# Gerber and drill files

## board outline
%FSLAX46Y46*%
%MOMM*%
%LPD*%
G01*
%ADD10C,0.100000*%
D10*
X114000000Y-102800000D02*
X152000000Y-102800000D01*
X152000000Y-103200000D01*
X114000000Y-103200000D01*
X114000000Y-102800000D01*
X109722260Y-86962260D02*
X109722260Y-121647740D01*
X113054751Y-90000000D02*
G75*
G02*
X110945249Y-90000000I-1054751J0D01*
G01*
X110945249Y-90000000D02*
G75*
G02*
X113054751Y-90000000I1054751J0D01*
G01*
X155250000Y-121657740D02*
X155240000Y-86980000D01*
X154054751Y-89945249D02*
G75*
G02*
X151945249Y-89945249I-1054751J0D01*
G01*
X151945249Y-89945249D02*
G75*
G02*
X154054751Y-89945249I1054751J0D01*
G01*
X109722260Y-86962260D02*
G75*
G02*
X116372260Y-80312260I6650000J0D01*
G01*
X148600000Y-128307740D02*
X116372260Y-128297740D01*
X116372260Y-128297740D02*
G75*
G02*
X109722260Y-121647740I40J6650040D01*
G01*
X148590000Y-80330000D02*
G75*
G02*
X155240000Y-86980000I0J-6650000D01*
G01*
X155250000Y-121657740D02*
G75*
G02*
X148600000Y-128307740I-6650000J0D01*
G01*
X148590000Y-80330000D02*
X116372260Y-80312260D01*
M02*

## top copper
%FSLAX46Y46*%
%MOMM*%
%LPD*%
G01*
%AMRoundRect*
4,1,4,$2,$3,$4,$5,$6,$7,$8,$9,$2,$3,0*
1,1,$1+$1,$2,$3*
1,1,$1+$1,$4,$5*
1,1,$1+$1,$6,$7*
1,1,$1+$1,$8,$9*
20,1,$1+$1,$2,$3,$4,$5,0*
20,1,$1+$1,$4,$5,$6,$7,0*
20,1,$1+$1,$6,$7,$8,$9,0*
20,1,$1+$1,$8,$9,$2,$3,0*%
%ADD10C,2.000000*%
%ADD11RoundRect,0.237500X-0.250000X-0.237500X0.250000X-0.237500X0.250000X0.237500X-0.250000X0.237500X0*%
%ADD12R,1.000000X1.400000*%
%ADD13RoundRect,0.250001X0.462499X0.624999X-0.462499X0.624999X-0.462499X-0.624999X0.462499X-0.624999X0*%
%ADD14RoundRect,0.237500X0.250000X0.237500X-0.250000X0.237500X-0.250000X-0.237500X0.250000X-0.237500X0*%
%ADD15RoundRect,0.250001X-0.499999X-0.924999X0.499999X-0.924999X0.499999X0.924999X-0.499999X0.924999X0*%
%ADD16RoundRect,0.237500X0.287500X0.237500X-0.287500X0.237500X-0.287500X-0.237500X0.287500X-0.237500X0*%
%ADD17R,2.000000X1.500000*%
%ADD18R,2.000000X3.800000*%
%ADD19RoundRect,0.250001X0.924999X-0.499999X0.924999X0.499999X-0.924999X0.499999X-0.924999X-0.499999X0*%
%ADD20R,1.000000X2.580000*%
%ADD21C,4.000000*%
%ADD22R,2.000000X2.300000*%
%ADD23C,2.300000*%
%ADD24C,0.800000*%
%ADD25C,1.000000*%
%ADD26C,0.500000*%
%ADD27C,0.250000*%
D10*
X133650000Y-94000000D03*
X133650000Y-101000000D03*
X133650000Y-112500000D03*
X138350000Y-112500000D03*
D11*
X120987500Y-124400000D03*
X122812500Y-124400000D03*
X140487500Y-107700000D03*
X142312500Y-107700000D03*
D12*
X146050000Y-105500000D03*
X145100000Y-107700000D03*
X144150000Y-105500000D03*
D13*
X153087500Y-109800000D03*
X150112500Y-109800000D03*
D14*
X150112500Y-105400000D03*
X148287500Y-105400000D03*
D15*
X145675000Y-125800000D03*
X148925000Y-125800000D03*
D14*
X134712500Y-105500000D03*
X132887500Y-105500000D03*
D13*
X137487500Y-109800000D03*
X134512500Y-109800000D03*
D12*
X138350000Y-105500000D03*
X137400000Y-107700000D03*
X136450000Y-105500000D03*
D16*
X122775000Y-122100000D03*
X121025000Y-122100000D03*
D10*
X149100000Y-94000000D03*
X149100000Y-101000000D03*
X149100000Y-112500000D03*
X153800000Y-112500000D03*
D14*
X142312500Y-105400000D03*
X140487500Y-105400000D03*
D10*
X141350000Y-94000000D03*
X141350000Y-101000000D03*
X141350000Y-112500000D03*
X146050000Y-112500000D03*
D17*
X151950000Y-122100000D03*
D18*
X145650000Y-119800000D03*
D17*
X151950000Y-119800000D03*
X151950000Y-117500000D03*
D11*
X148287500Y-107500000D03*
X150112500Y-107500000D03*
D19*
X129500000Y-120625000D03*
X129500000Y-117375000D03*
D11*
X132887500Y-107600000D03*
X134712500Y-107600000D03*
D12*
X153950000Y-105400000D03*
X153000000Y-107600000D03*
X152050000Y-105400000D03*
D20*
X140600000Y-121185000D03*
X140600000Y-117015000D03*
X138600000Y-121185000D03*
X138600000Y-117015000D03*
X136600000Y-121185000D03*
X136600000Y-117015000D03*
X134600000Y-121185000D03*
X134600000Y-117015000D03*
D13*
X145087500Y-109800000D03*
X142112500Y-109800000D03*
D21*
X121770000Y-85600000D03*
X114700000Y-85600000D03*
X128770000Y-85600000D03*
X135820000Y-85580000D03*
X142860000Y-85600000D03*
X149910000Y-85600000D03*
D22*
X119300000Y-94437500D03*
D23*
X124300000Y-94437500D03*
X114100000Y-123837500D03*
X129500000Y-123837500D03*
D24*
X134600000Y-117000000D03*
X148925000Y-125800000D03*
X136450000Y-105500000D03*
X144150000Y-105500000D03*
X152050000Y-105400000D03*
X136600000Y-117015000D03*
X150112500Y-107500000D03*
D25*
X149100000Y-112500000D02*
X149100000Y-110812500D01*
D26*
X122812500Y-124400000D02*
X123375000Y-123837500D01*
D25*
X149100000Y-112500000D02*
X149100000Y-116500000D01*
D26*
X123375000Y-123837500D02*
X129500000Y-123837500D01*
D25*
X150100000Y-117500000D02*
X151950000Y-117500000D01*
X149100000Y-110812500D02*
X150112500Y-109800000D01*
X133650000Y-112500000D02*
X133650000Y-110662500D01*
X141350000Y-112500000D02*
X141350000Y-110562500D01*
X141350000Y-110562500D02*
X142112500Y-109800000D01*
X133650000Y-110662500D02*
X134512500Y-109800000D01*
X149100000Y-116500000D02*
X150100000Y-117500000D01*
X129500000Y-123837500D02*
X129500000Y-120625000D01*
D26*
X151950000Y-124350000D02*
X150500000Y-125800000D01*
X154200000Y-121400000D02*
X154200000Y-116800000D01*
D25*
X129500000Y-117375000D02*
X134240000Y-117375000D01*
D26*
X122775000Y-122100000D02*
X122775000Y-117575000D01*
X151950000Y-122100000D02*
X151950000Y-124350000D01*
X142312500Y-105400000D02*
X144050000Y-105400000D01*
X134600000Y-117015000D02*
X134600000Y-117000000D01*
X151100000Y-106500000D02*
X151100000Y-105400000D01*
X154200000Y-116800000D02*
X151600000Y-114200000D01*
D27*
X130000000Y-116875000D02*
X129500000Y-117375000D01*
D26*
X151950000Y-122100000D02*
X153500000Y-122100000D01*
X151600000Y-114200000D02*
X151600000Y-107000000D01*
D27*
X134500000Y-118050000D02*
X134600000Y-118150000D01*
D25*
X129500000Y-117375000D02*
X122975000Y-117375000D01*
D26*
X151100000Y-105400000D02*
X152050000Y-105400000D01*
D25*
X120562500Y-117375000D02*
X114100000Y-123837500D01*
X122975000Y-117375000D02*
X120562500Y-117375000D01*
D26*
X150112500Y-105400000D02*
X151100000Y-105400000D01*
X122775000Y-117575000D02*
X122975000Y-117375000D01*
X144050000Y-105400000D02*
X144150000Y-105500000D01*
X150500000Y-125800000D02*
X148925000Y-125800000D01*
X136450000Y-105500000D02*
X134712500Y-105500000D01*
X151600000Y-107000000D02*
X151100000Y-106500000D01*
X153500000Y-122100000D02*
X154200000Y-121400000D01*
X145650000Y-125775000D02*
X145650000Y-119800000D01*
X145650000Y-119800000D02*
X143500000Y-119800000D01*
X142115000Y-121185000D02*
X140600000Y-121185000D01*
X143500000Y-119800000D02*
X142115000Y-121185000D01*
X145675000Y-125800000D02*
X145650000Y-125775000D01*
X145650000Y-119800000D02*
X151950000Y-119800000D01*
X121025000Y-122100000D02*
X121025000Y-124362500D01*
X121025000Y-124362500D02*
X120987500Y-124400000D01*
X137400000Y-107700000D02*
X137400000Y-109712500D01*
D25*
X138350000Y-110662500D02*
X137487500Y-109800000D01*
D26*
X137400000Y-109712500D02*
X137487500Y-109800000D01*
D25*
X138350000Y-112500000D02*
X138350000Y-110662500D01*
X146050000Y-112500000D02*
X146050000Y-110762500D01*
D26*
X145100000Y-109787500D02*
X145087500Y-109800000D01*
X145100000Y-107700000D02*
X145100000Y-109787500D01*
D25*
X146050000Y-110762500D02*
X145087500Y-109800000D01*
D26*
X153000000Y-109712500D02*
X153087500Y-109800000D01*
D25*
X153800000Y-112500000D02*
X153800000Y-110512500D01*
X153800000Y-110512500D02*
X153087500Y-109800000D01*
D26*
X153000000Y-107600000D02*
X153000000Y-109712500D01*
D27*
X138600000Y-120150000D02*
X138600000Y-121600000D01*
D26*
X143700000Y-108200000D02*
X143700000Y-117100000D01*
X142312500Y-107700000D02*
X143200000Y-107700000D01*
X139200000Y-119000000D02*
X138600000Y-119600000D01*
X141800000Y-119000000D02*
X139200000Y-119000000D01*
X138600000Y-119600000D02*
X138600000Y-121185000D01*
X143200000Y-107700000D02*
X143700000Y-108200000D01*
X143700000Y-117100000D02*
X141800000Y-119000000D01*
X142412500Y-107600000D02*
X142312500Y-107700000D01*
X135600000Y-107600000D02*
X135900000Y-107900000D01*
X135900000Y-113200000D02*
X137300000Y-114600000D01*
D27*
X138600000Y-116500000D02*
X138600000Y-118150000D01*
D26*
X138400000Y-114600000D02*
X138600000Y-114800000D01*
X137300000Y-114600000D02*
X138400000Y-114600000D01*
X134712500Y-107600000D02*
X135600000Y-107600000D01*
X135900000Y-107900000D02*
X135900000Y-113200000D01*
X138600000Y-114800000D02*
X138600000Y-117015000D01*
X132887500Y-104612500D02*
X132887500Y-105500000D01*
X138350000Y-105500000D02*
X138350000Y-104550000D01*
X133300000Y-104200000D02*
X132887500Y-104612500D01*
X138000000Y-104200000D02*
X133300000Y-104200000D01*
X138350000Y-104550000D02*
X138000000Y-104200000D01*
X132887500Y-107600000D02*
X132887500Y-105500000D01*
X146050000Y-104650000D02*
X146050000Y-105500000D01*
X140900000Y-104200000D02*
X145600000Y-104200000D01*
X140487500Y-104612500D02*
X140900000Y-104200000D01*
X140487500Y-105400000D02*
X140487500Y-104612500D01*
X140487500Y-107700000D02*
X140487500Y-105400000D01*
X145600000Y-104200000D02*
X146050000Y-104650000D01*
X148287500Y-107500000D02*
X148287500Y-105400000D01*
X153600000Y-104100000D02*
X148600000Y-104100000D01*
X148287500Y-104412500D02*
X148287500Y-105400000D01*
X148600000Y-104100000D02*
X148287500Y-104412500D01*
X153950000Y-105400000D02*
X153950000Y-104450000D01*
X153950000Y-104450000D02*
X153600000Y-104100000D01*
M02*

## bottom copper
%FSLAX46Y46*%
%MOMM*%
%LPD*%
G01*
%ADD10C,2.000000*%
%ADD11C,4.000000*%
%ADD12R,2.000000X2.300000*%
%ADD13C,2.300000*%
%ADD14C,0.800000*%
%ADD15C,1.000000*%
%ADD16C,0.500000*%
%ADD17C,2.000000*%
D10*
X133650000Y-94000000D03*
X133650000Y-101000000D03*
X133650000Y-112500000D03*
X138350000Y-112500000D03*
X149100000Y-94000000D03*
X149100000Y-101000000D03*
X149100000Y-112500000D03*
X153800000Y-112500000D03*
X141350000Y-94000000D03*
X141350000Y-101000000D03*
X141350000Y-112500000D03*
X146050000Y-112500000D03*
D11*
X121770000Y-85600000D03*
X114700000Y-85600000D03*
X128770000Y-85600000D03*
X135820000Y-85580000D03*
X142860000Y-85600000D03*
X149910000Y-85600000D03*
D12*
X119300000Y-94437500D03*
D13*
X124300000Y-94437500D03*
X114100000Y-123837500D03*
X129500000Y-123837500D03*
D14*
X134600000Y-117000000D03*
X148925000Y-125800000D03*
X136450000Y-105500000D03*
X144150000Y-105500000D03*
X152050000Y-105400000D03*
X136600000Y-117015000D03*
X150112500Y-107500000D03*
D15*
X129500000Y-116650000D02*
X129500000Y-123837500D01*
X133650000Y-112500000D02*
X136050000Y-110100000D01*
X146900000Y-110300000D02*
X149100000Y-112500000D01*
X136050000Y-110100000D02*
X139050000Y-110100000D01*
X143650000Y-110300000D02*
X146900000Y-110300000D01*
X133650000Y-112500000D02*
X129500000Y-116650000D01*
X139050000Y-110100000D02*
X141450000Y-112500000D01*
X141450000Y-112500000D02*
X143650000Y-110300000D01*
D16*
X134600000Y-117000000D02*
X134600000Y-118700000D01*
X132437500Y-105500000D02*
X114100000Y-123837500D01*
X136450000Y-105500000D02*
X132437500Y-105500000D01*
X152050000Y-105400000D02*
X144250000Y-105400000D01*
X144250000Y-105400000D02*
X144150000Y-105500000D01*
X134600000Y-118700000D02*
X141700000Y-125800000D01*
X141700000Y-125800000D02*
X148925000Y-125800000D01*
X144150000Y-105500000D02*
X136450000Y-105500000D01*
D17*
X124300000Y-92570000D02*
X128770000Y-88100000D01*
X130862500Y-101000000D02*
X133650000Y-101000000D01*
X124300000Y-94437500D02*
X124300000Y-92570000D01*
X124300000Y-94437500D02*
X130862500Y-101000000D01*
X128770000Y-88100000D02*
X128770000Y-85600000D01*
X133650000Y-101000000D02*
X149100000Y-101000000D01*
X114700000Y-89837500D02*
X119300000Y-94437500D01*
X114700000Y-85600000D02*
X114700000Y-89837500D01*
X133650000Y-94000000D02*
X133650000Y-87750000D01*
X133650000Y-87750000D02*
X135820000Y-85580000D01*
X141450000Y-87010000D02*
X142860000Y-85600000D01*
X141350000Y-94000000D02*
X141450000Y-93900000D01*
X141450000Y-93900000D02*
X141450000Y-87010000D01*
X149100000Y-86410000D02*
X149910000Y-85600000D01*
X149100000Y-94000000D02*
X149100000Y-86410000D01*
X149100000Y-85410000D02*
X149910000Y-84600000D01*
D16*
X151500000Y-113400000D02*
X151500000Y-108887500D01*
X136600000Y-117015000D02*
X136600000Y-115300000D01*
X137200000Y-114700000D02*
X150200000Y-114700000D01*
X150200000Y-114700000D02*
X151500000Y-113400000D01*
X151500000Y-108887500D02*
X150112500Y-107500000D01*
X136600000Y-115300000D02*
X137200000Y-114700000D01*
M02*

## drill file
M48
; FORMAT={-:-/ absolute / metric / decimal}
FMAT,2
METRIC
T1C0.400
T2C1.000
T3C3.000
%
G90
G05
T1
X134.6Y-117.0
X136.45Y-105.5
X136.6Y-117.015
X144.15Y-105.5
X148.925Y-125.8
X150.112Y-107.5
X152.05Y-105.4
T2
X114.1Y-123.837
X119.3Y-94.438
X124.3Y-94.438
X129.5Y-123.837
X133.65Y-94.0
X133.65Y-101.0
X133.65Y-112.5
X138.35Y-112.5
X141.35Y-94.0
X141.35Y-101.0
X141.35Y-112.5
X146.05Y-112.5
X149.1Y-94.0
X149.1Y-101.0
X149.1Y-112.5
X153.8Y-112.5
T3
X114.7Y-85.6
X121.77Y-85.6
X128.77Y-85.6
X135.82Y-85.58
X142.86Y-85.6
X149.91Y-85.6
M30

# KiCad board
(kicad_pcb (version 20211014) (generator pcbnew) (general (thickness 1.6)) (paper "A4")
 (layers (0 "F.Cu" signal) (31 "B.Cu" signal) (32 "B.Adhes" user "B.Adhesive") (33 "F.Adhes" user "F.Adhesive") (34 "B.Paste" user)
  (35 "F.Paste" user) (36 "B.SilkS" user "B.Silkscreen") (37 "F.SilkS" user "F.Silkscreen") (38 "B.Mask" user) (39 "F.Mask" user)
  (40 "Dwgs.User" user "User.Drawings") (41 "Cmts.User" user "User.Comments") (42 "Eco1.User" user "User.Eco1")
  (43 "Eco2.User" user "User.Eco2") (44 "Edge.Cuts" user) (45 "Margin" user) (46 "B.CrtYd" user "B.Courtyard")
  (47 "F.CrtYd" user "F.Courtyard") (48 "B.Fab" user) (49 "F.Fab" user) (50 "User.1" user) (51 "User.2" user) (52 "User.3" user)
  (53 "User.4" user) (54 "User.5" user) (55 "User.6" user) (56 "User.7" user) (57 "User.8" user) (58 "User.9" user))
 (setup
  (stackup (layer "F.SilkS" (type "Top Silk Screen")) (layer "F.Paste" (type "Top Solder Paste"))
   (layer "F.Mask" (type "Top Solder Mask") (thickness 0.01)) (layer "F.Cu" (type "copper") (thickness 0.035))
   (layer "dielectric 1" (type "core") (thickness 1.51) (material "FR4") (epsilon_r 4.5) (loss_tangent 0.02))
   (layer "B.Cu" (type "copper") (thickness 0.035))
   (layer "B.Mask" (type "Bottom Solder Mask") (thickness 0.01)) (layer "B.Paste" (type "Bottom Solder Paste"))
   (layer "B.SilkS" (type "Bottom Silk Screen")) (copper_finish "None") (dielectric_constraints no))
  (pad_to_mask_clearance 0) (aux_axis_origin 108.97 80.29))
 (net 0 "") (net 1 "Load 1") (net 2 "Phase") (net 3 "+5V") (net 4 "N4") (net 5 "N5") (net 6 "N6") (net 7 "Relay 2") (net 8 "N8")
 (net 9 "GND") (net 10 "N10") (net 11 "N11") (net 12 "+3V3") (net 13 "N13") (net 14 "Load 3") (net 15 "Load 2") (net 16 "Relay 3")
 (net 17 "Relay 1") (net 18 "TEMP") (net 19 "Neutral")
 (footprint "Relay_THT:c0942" (layer "F.Cu") (at 133.65 101 90)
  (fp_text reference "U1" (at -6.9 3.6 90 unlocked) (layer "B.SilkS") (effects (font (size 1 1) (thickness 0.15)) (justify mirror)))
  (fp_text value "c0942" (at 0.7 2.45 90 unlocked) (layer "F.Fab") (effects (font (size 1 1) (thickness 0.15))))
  (pad "1" thru_hole circle (at 7 0 90) (size 2 2) (drill 1) (layers *.Cu *.Mask) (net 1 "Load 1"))
  (pad "2" thru_hole circle (at 0 0 90) (size 2 2) (drill 1) (layers *.Cu *.Mask) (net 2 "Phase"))
  (pad "3" thru_hole circle (at -11.5 0 90) (size 2 2) (drill 1) (layers *.Cu *.Mask) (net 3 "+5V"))
  (pad "4" thru_hole circle (at -11.5 4.7 90) (size 2 2) (drill 1) (layers *.Cu *.Mask) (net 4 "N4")))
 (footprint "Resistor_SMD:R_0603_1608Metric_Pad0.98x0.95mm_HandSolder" (layer "F.Cu") (at 121.9 124.4)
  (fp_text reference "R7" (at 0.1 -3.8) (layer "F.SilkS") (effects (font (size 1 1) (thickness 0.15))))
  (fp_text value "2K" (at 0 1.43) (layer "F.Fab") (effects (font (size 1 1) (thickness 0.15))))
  (pad "1" smd roundrect (at -0.9125 0) (size 0.975 0.95) (layers "F.Cu" "F.Paste" "F.Mask") (roundrect_rratio 0.25) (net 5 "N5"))
  (pad "2" smd roundrect (at 0.9125 0) (size 0.975 0.95) (layers "F.Cu" "F.Paste" "F.Mask") (roundrect_rratio 0.25) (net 3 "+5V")))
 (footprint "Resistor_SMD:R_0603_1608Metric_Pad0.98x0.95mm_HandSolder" (layer "F.Cu") (at 141.4 107.7)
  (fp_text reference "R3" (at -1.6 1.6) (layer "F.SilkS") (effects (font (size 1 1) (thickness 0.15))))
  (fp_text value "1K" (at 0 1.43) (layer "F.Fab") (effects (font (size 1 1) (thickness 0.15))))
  (pad "1" smd roundrect (at -0.9125 0) (size 0.975 0.95) (layers "F.Cu" "F.Paste" "F.Mask") (roundrect_rratio 0.25) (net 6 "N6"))
  (pad "2" smd roundrect (at 0.9125 0) (size 0.975 0.95) (layers "F.Cu" "F.Paste" "F.Mask") (roundrect_rratio 0.25) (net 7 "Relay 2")))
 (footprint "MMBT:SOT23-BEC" (layer "F.Cu") (at 145.1 106.6 180)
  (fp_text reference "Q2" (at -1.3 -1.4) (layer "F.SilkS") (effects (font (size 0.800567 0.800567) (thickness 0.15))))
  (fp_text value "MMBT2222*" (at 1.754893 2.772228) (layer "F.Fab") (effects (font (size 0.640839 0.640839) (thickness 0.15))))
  (pad "B" smd rect locked (at -0.95 1.1 180) (size 1 1.4) (layers "F.Cu" "F.Paste" "F.Mask") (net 6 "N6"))
  (pad "C" smd rect locked (at 0 -1.1 180) (size 1 1.4) (layers "F.Cu" "F.Paste" "F.Mask") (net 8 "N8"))
  (pad "E" smd rect locked (at 0.95 1.1 180) (size 1 1.4) (layers "F.Cu" "F.Paste" "F.Mask") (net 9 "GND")))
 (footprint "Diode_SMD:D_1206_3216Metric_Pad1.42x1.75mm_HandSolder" (layer "F.Cu") (at 151.6 109.8 180)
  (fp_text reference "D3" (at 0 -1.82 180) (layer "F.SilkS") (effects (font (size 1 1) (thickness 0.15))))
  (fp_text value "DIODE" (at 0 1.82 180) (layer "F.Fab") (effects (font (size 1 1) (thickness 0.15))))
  (pad "1" smd roundrect (at -1.4875 0 180) (size 1.425 1.75) (layers "F.Cu" "F.Paste" "F.Mask") (roundrect_rratio 0.175439) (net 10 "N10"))
  (pad "2" smd roundrect (at 1.4875 0 180) (size 1.425 1.75) (layers "F.Cu" "F.Paste" "F.Mask") (roundrect_rratio 0.175439) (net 3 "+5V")))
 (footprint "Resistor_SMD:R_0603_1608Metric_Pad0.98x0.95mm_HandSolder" (layer "F.Cu") (at 149.2 105.4 180)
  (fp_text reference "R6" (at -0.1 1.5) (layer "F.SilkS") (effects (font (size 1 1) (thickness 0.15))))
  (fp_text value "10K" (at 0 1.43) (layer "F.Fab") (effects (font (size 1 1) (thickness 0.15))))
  (pad "1" smd roundrect (at -0.9125 0 180) (size 0.975 0.95) (layers "F.Cu" "F.Paste" "F.Mask") (roundrect_rratio 0.25) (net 9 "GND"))
  (pad "2" smd roundrect (at 0.9125 0 180) (size 0.975 0.95) (layers "F.Cu" "F.Paste" "F.Mask") (roundrect_rratio 0.25) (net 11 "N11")))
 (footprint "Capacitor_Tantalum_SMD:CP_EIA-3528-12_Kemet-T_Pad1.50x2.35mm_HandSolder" (layer "F.Cu") (at 147.3 125.8)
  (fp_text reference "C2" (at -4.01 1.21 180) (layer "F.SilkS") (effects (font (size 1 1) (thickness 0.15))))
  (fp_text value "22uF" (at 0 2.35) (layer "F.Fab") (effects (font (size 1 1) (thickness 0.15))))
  (pad "1" smd roundrect (at -1.625 0) (size 1.5 2.35) (layers "F.Cu" "F.Paste" "F.Mask") (roundrect_rratio 0.166667) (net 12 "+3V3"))
  (pad "2" smd roundrect (at 1.625 0) (size 1.5 2.35) (layers "F.Cu" "F.Paste" "F.Mask") (roundrect_rratio 0.166667) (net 9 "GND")))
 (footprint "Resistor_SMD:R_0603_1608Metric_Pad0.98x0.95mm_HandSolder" (layer "F.Cu") (at 133.8 105.5 180)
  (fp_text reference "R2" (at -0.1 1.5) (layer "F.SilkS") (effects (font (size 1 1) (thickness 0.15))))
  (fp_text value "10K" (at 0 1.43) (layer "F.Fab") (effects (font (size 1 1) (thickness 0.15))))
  (pad "1" smd roundrect (at -0.9125 0 180) (size 0.975 0.95) (layers "F.Cu" "F.Paste" "F.Mask") (roundrect_rratio 0.25) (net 9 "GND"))
  (pad "2" smd roundrect (at 0.9125 0 180) (size 0.975 0.95) (layers "F.Cu" "F.Paste" "F.Mask") (roundrect_rratio 0.25) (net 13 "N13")))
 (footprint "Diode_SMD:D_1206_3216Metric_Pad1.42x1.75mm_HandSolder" (layer "F.Cu") (at 136 109.8 180)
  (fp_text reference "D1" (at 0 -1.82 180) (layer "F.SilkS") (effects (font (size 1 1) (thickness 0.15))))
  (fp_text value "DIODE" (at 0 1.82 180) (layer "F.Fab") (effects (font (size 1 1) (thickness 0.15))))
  (pad "1" smd roundrect (at -1.4875 0 180) (size 1.425 1.75) (layers "F.Cu" "F.Paste" "F.Mask") (roundrect_rratio 0.175439) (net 4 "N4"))
  (pad "2" smd roundrect (at 1.4875 0 180) (size 1.425 1.75) (layers "F.Cu" "F.Paste" "F.Mask") (roundrect_rratio 0.175439) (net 3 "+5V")))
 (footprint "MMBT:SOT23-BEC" (layer "F.Cu") (at 137.4 106.6 180)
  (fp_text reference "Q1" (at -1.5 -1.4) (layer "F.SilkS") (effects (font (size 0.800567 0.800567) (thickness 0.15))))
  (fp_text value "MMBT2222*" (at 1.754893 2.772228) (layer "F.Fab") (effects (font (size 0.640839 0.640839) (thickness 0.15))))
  (pad "B" smd rect locked (at -0.95 1.1 180) (size 1 1.4) (layers "F.Cu" "F.Paste" "F.Mask") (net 13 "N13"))
  (pad "C" smd rect locked (at 0 -1.1 180) (size 1 1.4) (layers "F.Cu" "F.Paste" "F.Mask") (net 4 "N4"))
  (pad "E" smd rect locked (at 0.95 1.1 180) (size 1 1.4) (layers "F.Cu" "F.Paste" "F.Mask") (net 9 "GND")))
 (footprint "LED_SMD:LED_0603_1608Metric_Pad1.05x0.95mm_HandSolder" (layer "F.Cu") (at 121.9 122.1 180)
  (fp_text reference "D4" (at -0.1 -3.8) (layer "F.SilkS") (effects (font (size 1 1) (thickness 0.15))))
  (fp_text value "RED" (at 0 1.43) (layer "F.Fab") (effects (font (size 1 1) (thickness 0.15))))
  (pad "1" smd roundrect (at -0.875 0 180) (size 1.05 0.95) (layers "F.Cu" "F.Paste" "F.Mask") (roundrect_rratio 0.25) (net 9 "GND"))
  (pad "2" smd roundrect (at 0.875 0 180) (size 1.05 0.95) (layers "F.Cu" "F.Paste" "F.Mask") (roundrect_rratio 0.25) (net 5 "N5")))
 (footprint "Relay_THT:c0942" (layer "F.Cu") (at 149.1 101 90)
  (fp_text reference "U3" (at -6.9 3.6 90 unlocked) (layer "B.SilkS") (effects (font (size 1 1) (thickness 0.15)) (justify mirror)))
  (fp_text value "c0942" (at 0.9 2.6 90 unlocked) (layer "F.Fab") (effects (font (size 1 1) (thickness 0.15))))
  (pad "1" thru_hole circle (at 7 0 90) (size 2 2) (drill 1) (layers *.Cu *.Mask) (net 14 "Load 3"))
  (pad "2" thru_hole circle (at 0 0 90) (size 2 2) (drill 1) (layers *.Cu *.Mask) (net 2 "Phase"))
  (pad "3" thru_hole circle (at -11.5 0 90) (size 2 2) (drill 1) (layers *.Cu *.Mask) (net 3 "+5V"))
  (pad "4" thru_hole circle (at -11.5 4.7 90) (size 2 2) (drill 1) (layers *.Cu *.Mask) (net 10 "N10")))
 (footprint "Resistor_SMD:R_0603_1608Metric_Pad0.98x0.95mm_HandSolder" (layer "F.Cu") (at 141.4 105.4 180)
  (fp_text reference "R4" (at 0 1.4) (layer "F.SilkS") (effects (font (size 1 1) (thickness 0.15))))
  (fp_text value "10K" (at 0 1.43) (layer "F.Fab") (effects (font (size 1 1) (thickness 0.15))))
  (pad "1" smd roundrect (at -0.9125 0 180) (size 0.975 0.95) (layers "F.Cu" "F.Paste" "F.Mask") (roundrect_rratio 0.25) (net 9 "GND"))
  (pad "2" smd roundrect (at 0.9125 0 180) (size 0.975 0.95) (layers "F.Cu" "F.Paste" "F.Mask") (roundrect_rratio 0.25) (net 6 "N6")))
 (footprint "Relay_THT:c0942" (layer "F.Cu") (at 141.35 101 90)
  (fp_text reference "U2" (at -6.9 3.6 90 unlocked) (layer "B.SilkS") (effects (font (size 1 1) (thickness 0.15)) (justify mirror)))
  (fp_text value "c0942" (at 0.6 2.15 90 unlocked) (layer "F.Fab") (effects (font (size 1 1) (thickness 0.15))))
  (pad "1" thru_hole circle (at 7 0 90) (size 2 2) (drill 1) (layers *.Cu *.Mask) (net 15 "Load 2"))
  (pad "2" thru_hole circle (at 0 0 90) (size 2 2) (drill 1) (layers *.Cu *.Mask) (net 2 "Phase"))
  (pad "3" thru_hole circle (at -11.5 0 90) (size 2 2) (drill 1) (layers *.Cu *.Mask) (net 3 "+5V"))
  (pad "4" thru_hole circle (at -11.5 4.7 90) (size 2 2) (drill 1) (layers *.Cu *.Mask) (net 8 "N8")))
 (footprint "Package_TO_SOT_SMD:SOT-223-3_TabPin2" (layer "F.Cu") (at 148.8 119.8 180)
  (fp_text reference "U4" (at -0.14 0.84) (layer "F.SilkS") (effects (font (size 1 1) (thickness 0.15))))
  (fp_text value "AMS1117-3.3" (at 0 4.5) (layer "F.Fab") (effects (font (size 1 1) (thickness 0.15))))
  (pad "1" smd rect (at -3.15 -2.3 180) (size 2 1.5) (layers "F.Cu" "F.Paste" "F.Mask") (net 9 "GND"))
  (pad "2" smd rect (at 3.15 0 180) (size 2 3.8) (layers "F.Cu" "F.Paste" "F.Mask") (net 12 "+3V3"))
  (pad "2" smd rect (at -3.15 0 180) (size 2 1.5) (layers "F.Cu" "F.Paste" "F.Mask") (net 12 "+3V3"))
  (pad "3" smd rect (at -3.15 2.3 180) (size 2 1.5) (layers "F.Cu" "F.Paste" "F.Mask") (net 3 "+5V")))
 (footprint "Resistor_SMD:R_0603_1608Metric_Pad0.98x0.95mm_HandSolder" (layer "F.Cu") (at 149.2 107.5)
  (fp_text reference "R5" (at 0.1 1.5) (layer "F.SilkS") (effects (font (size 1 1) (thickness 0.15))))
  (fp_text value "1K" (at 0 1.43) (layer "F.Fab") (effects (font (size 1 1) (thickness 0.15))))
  (pad "1" smd roundrect (at -0.9125 0) (size 0.975 0.95) (layers "F.Cu" "F.Paste" "F.Mask") (roundrect_rratio 0.25) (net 11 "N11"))
  (pad "2" smd roundrect (at 0.9125 0) (size 0.975 0.95) (layers "F.Cu" "F.Paste" "F.Mask") (roundrect_rratio 0.25) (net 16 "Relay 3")))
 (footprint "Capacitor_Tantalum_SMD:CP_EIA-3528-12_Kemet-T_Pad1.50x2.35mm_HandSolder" (layer "F.Cu") (at 129.5 119 90)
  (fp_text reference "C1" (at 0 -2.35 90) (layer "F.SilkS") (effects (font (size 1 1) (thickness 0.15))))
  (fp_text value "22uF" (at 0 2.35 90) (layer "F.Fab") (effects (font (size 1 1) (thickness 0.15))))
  (pad "1" smd roundrect (at -1.625 0 90) (size 1.5 2.35) (layers "F.Cu" "F.Paste" "F.Mask") (roundrect_rratio 0.166667) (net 3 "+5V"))
  (pad "2" smd roundrect (at 1.625 0 90) (size 1.5 2.35) (layers "F.Cu" "F.Paste" "F.Mask") (roundrect_rratio 0.166667) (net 9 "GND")))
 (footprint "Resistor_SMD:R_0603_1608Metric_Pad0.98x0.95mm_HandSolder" (layer "F.Cu") (at 133.8 107.6)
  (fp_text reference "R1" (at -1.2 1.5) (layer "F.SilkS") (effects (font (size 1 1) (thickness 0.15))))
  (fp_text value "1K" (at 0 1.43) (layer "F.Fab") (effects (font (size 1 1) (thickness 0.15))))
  (pad "1" smd roundrect (at -0.9125 0) (size 0.975 0.95) (layers "F.Cu" "F.Paste" "F.Mask") (roundrect_rratio 0.25) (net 13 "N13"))
  (pad "2" smd roundrect (at 0.9125 0) (size 0.975 0.95) (layers "F.Cu" "F.Paste" "F.Mask") (roundrect_rratio 0.25) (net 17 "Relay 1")))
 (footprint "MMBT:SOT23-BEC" (layer "F.Cu") (at 153 106.5 180)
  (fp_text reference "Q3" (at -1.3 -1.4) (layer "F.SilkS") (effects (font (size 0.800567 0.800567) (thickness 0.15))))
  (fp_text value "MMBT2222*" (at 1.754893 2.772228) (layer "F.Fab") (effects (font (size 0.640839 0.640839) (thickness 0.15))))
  (pad "B" smd rect locked (at -0.95 1.1 180) (size 1 1.4) (layers "F.Cu" "F.Paste" "F.Mask") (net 11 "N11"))
  (pad "C" smd rect locked (at 0 -1.1 180) (size 1 1.4) (layers "F.Cu" "F.Paste" "F.Mask") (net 10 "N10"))
  (pad "E" smd rect locked (at 0.95 1.1 180) (size 1 1.4) (layers "F.Cu" "F.Paste" "F.Mask") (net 9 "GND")))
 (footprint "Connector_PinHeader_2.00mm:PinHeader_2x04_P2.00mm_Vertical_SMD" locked (layer "F.Cu") (at 137.6 119.1 -90)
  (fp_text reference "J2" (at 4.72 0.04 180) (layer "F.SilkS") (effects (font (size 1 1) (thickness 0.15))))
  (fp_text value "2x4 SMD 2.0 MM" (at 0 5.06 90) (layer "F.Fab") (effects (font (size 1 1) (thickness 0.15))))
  (pad "1" smd rect locked (at 2.085 -3 270) (size 2.58 1) (layers "F.Cu" "F.Paste" "F.Mask") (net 12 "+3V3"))
  (pad "2" smd rect locked (at -2.085 -3 270) (size 2.58 1) (layers "F.Cu" "F.Paste" "F.Mask"))
  (pad "3" smd rect locked (at 2.085 -1 270) (size 2.58 1) (layers "F.Cu" "F.Paste" "F.Mask") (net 7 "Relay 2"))
  (pad "4" smd rect locked (at -2.085 -1 270) (size 2.58 1) (layers "F.Cu" "F.Paste" "F.Mask") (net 17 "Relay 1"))
  (pad "5" smd rect locked (at 2.085 1 270) (size 2.58 1) (layers "F.Cu" "F.Paste" "F.Mask"))
  (pad "6" smd rect locked (at -2.085 1 270) (size 2.58 1) (layers "F.Cu" "F.Paste" "F.Mask") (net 16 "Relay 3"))
  (pad "7" smd rect locked (at 2.085 3 270) (size 2.58 1) (layers "F.Cu" "F.Paste" "F.Mask") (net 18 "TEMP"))
  (pad "8" smd rect locked (at -2.085 3 270) (size 2.58 1) (layers "F.Cu" "F.Paste" "F.Mask") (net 9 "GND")))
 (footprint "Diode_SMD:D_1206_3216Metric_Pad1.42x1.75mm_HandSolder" (layer "F.Cu") (at 143.6 109.8 180)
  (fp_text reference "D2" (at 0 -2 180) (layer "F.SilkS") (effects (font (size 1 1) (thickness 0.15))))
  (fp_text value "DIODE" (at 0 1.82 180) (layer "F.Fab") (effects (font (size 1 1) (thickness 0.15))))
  (pad "1" smd roundrect (at -1.4875 0 180) (size 1.425 1.75) (layers "F.Cu" "F.Paste" "F.Mask") (roundrect_rratio 0.175439) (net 8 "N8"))
  (pad "2" smd roundrect (at 1.4875 0 180) (size 1.425 1.75) (layers "F.Cu" "F.Paste" "F.Mask") (roundrect_rratio 0.175439) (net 3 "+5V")))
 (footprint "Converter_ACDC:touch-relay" (layer "B.Cu") (at 114.7 85.6 90)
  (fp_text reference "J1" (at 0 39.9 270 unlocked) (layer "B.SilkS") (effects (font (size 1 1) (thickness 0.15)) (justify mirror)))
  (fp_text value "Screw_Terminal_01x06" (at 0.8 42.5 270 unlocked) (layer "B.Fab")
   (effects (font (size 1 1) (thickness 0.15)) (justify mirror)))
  (pad "1" thru_hole circle (at 0 7.07 90) (size 4 4) (drill 3) (layers *.Cu *.Mask))
  (pad "2" thru_hole circle (at 0 0 90) (size 4 4) (drill 3) (layers *.Cu *.Mask) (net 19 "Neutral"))
  (pad "3" thru_hole circle (at 0 14.07 90) (size 4 4) (drill 3) (layers *.Cu *.Mask) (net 2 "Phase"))
  (pad "4" thru_hole circle (at 0.02 21.12 90) (size 4 4) (drill 3) (layers *.Cu *.Mask) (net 1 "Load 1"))
  (pad "5" thru_hole circle (at 0 28.16 90) (size 4 4) (drill 3) (layers *.Cu *.Mask) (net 15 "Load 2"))
  (pad "6" thru_hole circle (at 0 35.21 90) (size 4 4) (drill 3) (layers *.Cu *.Mask) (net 14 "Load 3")))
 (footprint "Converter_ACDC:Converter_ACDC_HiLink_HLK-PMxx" (layer "B.Cu") (at 119.3 94.4375 -90)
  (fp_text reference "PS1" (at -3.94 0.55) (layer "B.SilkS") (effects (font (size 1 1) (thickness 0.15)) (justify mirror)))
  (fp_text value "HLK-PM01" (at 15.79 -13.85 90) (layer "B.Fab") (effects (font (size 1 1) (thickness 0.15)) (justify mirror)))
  (pad "1" thru_hole rect (at 0 0 270) (size 2.3 2) (drill 1) (layers *.Cu *.Mask) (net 19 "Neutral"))
  (pad "2" thru_hole circle (at 0 -5 270) (size 2.3 2.3) (drill 1) (layers *.Cu *.Mask) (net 2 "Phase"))
  (pad "3" thru_hole circle (at 29.4 5.2 270) (size 2.3 2.3) (drill 1) (layers *.Cu *.Mask) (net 9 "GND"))
  (pad "4" thru_hole circle (at 29.4 -10.2 270) (size 2.3 2.3) (drill 1) (layers *.Cu *.Mask) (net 3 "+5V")))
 (gr_rect (start 152 102.8) (end 114 103.2) (layer "Edge.Cuts") (width 0.1) (fill none))
 (gr_line (start 109.72226 86.96226) (end 109.72226 121.64774) (layer "Edge.Cuts") (width 0.1))
 (gr_circle (center 112 90) (end 111.1 89.45) (layer "Edge.Cuts") (width 0.1) (fill none))
 (gr_line (start 155.25 121.65774) (end 155.24 86.98) (layer "Edge.Cuts") (width 0.1))
 (gr_circle (center 153 89.945249) (end 152.1 89.395249) (layer "Edge.Cuts") (width 0.1) (fill none))
 (gr_arc (start 109.72226 86.96226) (mid 111.67 82.26) (end 116.37226 80.31226) (layer "Edge.Cuts") (width 0.1))
 (gr_line (start 148.6 128.30774) (end 116.37226 128.29774) (layer "Edge.Cuts") (width 0.1))
 (gr_arc (start 116.37226 128.29774) (mid 111.67 126.35) (end 109.72226 121.64774) (layer "Edge.Cuts") (width 0.1))
 (gr_arc (start 148.59 80.33) (mid 153.29226 82.27774) (end 155.24 86.98) (layer "Edge.Cuts") (width 0.1))
 (gr_arc (start 155.25 121.65774) (mid 153.30226 126.36) (end 148.6 128.30774) (layer "Edge.Cuts") (width 0.1))
 (gr_line (start 148.59 80.33) (end 116.37226 80.31226) (layer "Edge.Cuts") (width 0.1))
 (segment (start 149.1 112.5) (end 149.1 110.8125) (width 1) (layer "F.Cu") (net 3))
 (segment (start 122.8125 124.4) (end 123.375 123.8375) (width 0.5) (layer "F.Cu") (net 3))
 (segment (start 149.1 112.5) (end 149.1 116.5) (width 1) (layer "F.Cu") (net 3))
 (segment (start 123.375 123.8375) (end 129.5 123.8375) (width 0.5) (layer "F.Cu") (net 3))
 (segment (start 150.1 117.5) (end 151.95 117.5) (width 1) (layer "F.Cu") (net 3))
 (segment (start 149.1 110.8125) (end 150.1125 109.8) (width 1) (layer "F.Cu") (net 3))
 (segment (start 133.65 112.5) (end 133.65 110.6625) (width 1) (layer "F.Cu") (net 3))
 (segment (start 141.35 112.5) (end 141.35 110.5625) (width 1) (layer "F.Cu") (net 3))
 (segment (start 141.35 110.5625) (end 142.1125 109.8) (width 1) (layer "F.Cu") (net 3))
 (segment (start 133.65 110.6625) (end 134.5125 109.8) (width 1) (layer "F.Cu") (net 3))
 (segment (start 149.1 116.5) (end 150.1 117.5) (width 1) (layer "F.Cu") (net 3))
 (segment (start 129.5 123.8375) (end 129.5 120.625) (width 1) (layer "F.Cu") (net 3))
 (segment (start 129.5 116.65) (end 129.5 123.8375) (width 1) (layer "B.Cu") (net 3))
 (segment (start 133.65 112.5) (end 136.05 110.1) (width 1) (layer "B.Cu") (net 3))
 (segment (start 146.9 110.3) (end 149.1 112.5) (width 1) (layer "B.Cu") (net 3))
 (segment (start 136.05 110.1) (end 139.05 110.1) (width 1) (layer "B.Cu") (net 3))
 (segment (start 143.65 110.3) (end 146.9 110.3) (width 1) (layer "B.Cu") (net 3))
 (segment (start 133.65 112.5) (end 129.5 116.65) (width 1) (layer "B.Cu") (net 3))
 (segment (start 139.05 110.1) (end 141.45 112.5) (width 1) (layer "B.Cu") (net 3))
 (segment (start 141.45 112.5) (end 143.65 110.3) (width 1) (layer "B.Cu") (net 3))
 (segment (start 151.95 124.35) (end 150.5 125.8) (width 0.5) (layer "F.Cu") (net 9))
 (segment (start 154.2 121.4) (end 154.2 116.8) (width 0.5) (layer "F.Cu") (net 9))
 (segment (start 129.5 117.375) (end 134.24 117.375) (width 1) (layer "F.Cu") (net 9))
 (segment (start 122.775 122.1) (end 122.775 117.575) (width 0.5) (layer "F.Cu") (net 9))
 (segment (start 151.95 122.1) (end 151.95 124.35) (width 0.5) (layer "F.Cu") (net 9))
 (segment (start 142.3125 105.4) (end 144.05 105.4) (width 0.5) (layer "F.Cu") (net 9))
 (segment (start 134.6 117.015) (end 134.6 117) (width 0.5) (layer "F.Cu") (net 9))
 (segment (start 151.1 106.5) (end 151.1 105.4) (width 0.5) (layer "F.Cu") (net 9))
 (segment (start 154.2 116.8) (end 151.6 114.2) (width 0.5) (layer "F.Cu") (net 9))
 (segment (start 130 116.875) (end 129.5 117.375) (width 0.25) (layer "F.Cu") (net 9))
 (segment (start 151.95 122.1) (end 153.5 122.1) (width 0.5) (layer "F.Cu") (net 9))
 (segment (start 151.6 114.2) (end 151.6 107) (width 0.5) (layer "F.Cu") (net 9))
 (segment (start 134.5 118.05) (end 134.6 118.15) (width 0.25) (layer "F.Cu") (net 9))
 (segment (start 129.5 117.375) (end 122.975 117.375) (width 1) (layer "F.Cu") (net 9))
 (segment (start 151.1 105.4) (end 152.05 105.4) (width 0.5) (layer "F.Cu") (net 9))
 (segment (start 120.5625 117.375) (end 114.1 123.8375) (width 1) (layer "F.Cu") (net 9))
 (segment (start 122.975 117.375) (end 120.5625 117.375) (width 1) (layer "F.Cu") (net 9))
 (segment (start 150.1125 105.4) (end 151.1 105.4) (width 0.5) (layer "F.Cu") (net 9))
 (segment (start 122.775 117.575) (end 122.975 117.375) (width 0.5) (layer "F.Cu") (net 9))
 (segment (start 144.05 105.4) (end 144.15 105.5) (width 0.5) (layer "F.Cu") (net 9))
 (segment (start 150.5 125.8) (end 148.925 125.8) (width 0.5) (layer "F.Cu") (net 9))
 (segment (start 136.45 105.5) (end 134.7125 105.5) (width 0.5) (layer "F.Cu") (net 9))
 (segment (start 151.6 107) (end 151.1 106.5) (width 0.5) (layer "F.Cu") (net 9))
 (segment (start 153.5 122.1) (end 154.2 121.4) (width 0.5) (layer "F.Cu") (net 9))
 (via (at 134.6 117) (size 0.8) (drill 0.4) (layers "F.Cu" "B.Cu") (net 9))
 (via (at 148.925 125.8) (size 0.8) (drill 0.4) (layers "F.Cu" "B.Cu") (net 9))
 (via (at 136.45 105.5) (size 0.8) (drill 0.4) (layers "F.Cu" "B.Cu") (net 9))
 (via (at 144.15 105.5) (size 0.8) (drill 0.4) (layers "F.Cu" "B.Cu") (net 9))
 (via (at 152.05 105.4) (size 0.8) (drill 0.4) (layers "F.Cu" "B.Cu") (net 9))
 (segment (start 134.6 117) (end 134.6 118.7) (width 0.5) (layer "B.Cu") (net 9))
 (segment (start 132.4375 105.5) (end 114.1 123.8375) (width 0.5) (layer "B.Cu") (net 9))
 (segment (start 136.45 105.5) (end 132.4375 105.5) (width 0.5) (layer "B.Cu") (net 9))
 (segment (start 152.05 105.4) (end 144.25 105.4) (width 0.5) (layer "B.Cu") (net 9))
 (segment (start 144.25 105.4) (end 144.15 105.5) (width 0.5) (layer "B.Cu") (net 9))
 (segment (start 134.6 118.7) (end 141.7 125.8) (width 0.5) (layer "B.Cu") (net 9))
 (segment (start 141.7 125.8) (end 148.925 125.8) (width 0.5) (layer "B.Cu") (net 9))
 (segment (start 144.15 105.5) (end 136.45 105.5) (width 0.5) (layer "B.Cu") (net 9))
 (segment (start 145.65 125.775) (end 145.65 119.8) (width 0.5) (layer "F.Cu") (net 12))
 (segment (start 145.65 119.8) (end 143.5 119.8) (width 0.5) (layer "F.Cu") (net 12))
 (segment (start 142.115 121.185) (end 140.6 121.185) (width 0.5) (layer "F.Cu") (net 12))
 (segment (start 143.5 119.8) (end 142.115 121.185) (width 0.5) (layer "F.Cu") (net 12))
 (segment (start 145.675 125.8) (end 145.65 125.775) (width 0.5) (layer "F.Cu") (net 12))
 (segment (start 145.65 119.8) (end 151.95 119.8) (width 0.5) (layer "F.Cu") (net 12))
 (segment (start 121.025 122.1) (end 121.025 124.3625) (width 0.5) (layer "F.Cu") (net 5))
 (segment (start 121.025 124.3625) (end 120.9875 124.4) (width 0.5) (layer "F.Cu") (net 5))
 (segment (start 124.3 92.57) (end 128.77 88.1) (width 2) (layer "B.Cu") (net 2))
 (segment (start 130.8625 101) (end 133.65 101) (width 2) (layer "B.Cu") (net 2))
 (segment (start 124.3 94.4375) (end 124.3 92.57) (width 2) (layer "B.Cu") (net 2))
 (segment (start 124.3 94.4375) (end 130.8625 101) (width 2) (layer "B.Cu") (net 2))
 (segment (start 128.77 88.1) (end 128.77 85.6) (width 2) (layer "B.Cu") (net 2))
 (segment (start 133.65 101) (end 149.1 101) (width 2) (layer "B.Cu") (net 2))
 (segment (start 137.4 107.7) (end 137.4 109.7125) (width 0.5) (layer "F.Cu") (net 4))
 (segment (start 138.35 110.6625) (end 137.4875 109.8) (width 1) (layer "F.Cu") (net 4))
 (segment (start 137.4 109.7125) (end 137.4875 109.8) (width 0.5) (layer "F.Cu") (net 4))
 (segment (start 138.35 112.5) (end 138.35 110.6625) (width 1) (layer "F.Cu") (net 4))
 (segment (start 146.05 112.5) (end 146.05 110.7625) (width 1) (layer "F.Cu") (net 8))
 (segment (start 145.1 109.7875) (end 145.0875 109.8) (width 0.5) (layer "F.Cu") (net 8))
 (segment (start 145.1 107.7) (end 145.1 109.7875) (width 0.5) (layer "F.Cu") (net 8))
 (segment (start 146.05 110.7625) (end 145.0875 109.8) (width 1) (layer "F.Cu") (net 8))
 (segment (start 153 109.7125) (end 153.0875 109.8) (width 0.5) (layer "F.Cu") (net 10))
 (segment (start 153.8 112.5) (end 153.8 110.5125) (width 1) (layer "F.Cu") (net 10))
 (segment (start 153.8 110.5125) (end 153.0875 109.8) (width 1) (layer "F.Cu") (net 10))
 (segment (start 153 107.6) (end 153 109.7125) (width 0.5) (layer "F.Cu") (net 10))
 (segment (start 114.7 89.8375) (end 119.3 94.4375) (width 2) (layer "B.Cu") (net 19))
 (segment (start 114.7 85.6) (end 114.7 89.8375) (width 2) (layer "B.Cu") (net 19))
 (segment (start 133.65 94) (end 133.65 87.75) (width 2) (layer "B.Cu") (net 1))
 (segment (start 133.65 87.75) (end 135.82 85.58) (width 2) (layer "B.Cu") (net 1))
 (segment (start 141.45 87.01) (end 142.86 85.6) (width 2) (layer "B.Cu") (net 15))
 (segment (start 141.35 94) (end 141.45 93.9) (width 2) (layer "B.Cu") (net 15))
 (segment (start 141.45 93.9) (end 141.45 87.01) (width 2) (layer "B.Cu") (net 15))
 (segment (start 149.1 86.41) (end 149.91 85.6) (width 2) (layer "B.Cu") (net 14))
 (segment (start 149.1 94) (end 149.1 86.41) (width 2) (layer "B.Cu") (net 14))
 (segment (start 149.1 85.41) (end 149.91 84.6) (width 2) (layer "B.Cu") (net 14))
 (segment (start 138.6 120.15) (end 138.6 121.6) (width 0.25) (layer "F.Cu") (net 7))
 (segment (start 143.7 108.2) (end 143.7 117.1) (width 0.5) (layer "F.Cu") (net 7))
 (segment (start 142.3125 107.7) (end 143.2 107.7) (width 0.5) (layer "F.Cu") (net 7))
 (segment (start 139.2 119) (end 138.6 119.6) (width 0.5) (layer "F.Cu") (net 7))
 (segment (start 141.8 119) (end 139.2 119) (width 0.5) (layer "F.Cu") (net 7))
 (segment (start 138.6 119.6) (end 138.6 121.185) (width 0.5) (layer "F.Cu") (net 7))
 (segment (start 143.2 107.7) (end 143.7 108.2) (width 0.5) (layer "F.Cu") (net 7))
 (segment (start 143.7 117.1) (end 141.8 119) (width 0.5) (layer "F.Cu") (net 7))
 (segment (start 142.4125 107.6) (end 142.3125 107.7) (width 0.5) (layer "F.Cu") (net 7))
 (segment (start 135.6 107.6) (end 135.9 107.9) (width 0.5) (layer "F.Cu") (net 17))
 (segment (start 135.9 113.2) (end 137.3 114.6) (width 0.5) (layer "F.Cu") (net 17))
 (segment (start 138.6 116.5) (end 138.6 118.15) (width 0.25) (layer "F.Cu") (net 17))
 (segment (start 138.4 114.6) (end 138.6 114.8) (width 0.5) (layer "F.Cu") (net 17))
 (segment (start 137.3 114.6) (end 138.4 114.6) (width 0.5) (layer "F.Cu") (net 17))
 (segment (start 134.7125 107.6) (end 135.6 107.6) (width 0.5) (layer "F.Cu") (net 17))
 (segment (start 135.9 107.9) (end 135.9 113.2) (width 0.5) (layer "F.Cu") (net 17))
 (segment (start 138.6 114.8) (end 138.6 117.015) (width 0.5) (layer "F.Cu") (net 17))
 (via (at 136.6 117.015) (size 0.8) (drill 0.4) (layers "F.Cu" "B.Cu") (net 16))
 (via (at 150.1125 107.5) (size 0.8) (drill 0.4) (layers "F.Cu" "B.Cu") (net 16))
 (segment (start 151.5 113.4) (end 151.5 108.8875) (width 0.5) (layer "B.Cu") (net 16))
 (segment (start 136.6 117.015) (end 136.6 115.3) (width 0.5) (layer "B.Cu") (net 16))
 (segment (start 137.2 114.7) (end 150.2 114.7) (width 0.5) (layer "B.Cu") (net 16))
 (segment (start 150.2 114.7) (end 151.5 113.4) (width 0.5) (layer "B.Cu") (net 16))
 (segment (start 151.5 108.8875) (end 150.1125 107.5) (width 0.5) (layer "B.Cu") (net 16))
 (segment (start 136.6 115.3) (end 137.2 114.7) (width 0.5) (layer "B.Cu") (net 16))
 (segment (start 132.8875 104.6125) (end 132.8875 105.5) (width 0.5) (layer "F.Cu") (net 13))
 (segment (start 138.35 105.5) (end 138.35 104.55) (width 0.5) (layer "F.Cu") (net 13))
 (segment (start 133.3 104.2) (end 132.8875 104.6125) (width 0.5) (layer "F.Cu") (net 13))
 (segment (start 138 104.2) (end 133.3 104.2) (width 0.5) (layer "F.Cu") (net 13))
 (segment (start 138.35 104.55) (end 138 104.2) (width 0.5) (layer "F.Cu") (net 13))
 (segment (start 132.8875 107.6) (end 132.8875 105.5) (width 0.5) (layer "F.Cu") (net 13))
 (segment (start 146.05 104.65) (end 146.05 105.5) (width 0.5) (layer "F.Cu") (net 6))
 (segment (start 140.9 104.2) (end 145.6 104.2) (width 0.5) (layer "F.Cu") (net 6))
 (segment (start 140.4875 104.6125) (end 140.9 104.2) (width 0.5) (layer "F.Cu") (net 6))
 (segment (start 140.4875 105.4) (end 140.4875 104.6125) (width 0.5) (layer "F.Cu") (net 6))
 (segment (start 140.4875 107.7) (end 140.4875 105.4) (width 0.5) (layer "F.Cu") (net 6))
 (segment (start 145.6 104.2) (end 146.05 104.65) (width 0.5) (layer "F.Cu") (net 6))
 (segment (start 148.2875 107.5) (end 148.2875 105.4) (width 0.5) (layer "F.Cu") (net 11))
 (segment (start 153.6 104.1) (end 148.6 104.1) (width 0.5) (layer "F.Cu") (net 11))
 (segment (start 148.2875 104.4125) (end 148.2875 105.4) (width 0.5) (layer "F.Cu") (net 11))
 (segment (start 148.6 104.1) (end 148.2875 104.4125) (width 0.5) (layer "F.Cu") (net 11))
 (segment (start 153.95 105.4) (end 153.95 104.45) (width 0.5) (layer "F.Cu") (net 11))
 (segment (start 153.95 104.45) (end 153.6 104.1) (width 0.5) (layer "F.Cu") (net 11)))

